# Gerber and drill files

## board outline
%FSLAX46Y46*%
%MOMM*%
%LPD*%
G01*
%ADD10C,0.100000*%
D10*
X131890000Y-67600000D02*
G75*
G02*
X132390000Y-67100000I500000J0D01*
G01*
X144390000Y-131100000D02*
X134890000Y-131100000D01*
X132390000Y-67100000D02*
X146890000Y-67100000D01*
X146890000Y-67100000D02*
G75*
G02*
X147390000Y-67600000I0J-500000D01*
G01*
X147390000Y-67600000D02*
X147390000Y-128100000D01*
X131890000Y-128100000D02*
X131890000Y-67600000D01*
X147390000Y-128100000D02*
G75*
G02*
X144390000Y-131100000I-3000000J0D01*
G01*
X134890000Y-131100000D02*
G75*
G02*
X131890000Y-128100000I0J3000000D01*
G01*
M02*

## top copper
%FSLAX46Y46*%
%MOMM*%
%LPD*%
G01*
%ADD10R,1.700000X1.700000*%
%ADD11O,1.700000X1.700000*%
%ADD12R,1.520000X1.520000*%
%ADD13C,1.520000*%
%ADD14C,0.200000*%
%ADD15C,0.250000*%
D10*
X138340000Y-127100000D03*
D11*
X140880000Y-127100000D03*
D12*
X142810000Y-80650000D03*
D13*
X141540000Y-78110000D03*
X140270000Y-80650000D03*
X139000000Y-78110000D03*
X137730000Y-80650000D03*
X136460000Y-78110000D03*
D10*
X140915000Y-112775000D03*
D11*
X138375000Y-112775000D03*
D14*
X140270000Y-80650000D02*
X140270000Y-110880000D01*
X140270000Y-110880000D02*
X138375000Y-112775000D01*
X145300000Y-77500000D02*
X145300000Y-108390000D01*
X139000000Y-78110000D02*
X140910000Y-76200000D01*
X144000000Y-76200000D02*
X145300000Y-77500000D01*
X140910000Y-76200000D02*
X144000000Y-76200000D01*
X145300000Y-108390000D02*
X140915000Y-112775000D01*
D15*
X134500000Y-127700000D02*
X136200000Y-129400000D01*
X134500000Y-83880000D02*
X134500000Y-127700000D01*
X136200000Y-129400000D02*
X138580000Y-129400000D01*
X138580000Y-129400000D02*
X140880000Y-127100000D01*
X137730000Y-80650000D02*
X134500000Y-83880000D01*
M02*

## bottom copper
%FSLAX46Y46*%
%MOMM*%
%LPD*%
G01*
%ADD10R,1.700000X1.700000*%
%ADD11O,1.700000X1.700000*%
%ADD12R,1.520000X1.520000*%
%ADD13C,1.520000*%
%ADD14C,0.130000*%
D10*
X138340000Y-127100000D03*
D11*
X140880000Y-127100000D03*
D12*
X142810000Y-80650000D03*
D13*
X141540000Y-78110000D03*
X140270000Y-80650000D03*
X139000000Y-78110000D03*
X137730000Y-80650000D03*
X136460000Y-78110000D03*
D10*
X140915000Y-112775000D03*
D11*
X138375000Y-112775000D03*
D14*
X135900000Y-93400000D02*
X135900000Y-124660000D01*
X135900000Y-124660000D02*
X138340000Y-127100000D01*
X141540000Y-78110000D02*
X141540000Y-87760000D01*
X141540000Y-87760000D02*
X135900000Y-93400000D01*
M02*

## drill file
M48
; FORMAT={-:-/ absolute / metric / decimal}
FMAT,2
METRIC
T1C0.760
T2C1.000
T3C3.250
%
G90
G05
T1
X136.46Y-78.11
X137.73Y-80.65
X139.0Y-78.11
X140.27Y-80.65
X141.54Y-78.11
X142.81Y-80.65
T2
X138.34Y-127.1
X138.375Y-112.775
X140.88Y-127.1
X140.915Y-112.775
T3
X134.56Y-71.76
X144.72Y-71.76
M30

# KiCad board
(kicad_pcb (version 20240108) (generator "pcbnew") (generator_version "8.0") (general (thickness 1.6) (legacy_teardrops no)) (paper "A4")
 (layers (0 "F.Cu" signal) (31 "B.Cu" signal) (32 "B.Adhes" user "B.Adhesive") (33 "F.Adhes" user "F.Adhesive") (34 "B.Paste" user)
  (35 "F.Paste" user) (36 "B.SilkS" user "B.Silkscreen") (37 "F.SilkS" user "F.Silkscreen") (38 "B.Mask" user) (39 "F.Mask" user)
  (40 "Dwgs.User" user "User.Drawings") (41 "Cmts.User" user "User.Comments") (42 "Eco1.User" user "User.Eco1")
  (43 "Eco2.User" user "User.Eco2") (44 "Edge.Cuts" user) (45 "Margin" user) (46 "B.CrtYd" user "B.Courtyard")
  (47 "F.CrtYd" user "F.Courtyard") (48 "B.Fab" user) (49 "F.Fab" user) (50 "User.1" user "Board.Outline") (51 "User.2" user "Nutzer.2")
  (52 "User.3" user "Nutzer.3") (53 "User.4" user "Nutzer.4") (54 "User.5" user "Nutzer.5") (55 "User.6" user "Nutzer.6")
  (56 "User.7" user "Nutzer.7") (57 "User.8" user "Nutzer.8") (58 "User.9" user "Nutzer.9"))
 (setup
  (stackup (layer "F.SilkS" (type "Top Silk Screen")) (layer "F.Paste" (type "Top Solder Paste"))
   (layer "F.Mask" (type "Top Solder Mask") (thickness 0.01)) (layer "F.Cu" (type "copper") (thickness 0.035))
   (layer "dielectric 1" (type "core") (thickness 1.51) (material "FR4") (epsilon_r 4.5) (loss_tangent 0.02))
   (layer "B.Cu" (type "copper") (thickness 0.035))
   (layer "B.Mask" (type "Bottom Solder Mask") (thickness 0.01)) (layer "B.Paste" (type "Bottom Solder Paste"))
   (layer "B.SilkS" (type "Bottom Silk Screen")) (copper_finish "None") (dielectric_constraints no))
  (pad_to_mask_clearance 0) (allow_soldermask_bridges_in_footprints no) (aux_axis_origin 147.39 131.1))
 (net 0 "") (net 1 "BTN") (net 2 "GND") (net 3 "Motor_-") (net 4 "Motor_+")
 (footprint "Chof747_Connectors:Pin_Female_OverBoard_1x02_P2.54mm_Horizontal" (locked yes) (layer "F.Cu") (at 138.34 127.1 90)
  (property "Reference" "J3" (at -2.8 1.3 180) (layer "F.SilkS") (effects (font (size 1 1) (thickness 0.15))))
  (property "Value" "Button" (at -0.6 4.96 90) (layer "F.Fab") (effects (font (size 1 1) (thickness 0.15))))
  (pad "1" thru_hole rect (at 0 0 90) (size 1.7 1.7) (drill 1) (layers "*.Cu" "*.Mask") (remove_unused_layers no) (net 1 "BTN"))
  (pad "2" thru_hole oval (at 0 2.54 90) (size 1.7 1.7) (drill 1) (layers "*.Cu" "*.Mask") (remove_unused_layers no) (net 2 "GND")))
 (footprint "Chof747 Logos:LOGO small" (layer "F.Cu") (at 135.099998 91.5)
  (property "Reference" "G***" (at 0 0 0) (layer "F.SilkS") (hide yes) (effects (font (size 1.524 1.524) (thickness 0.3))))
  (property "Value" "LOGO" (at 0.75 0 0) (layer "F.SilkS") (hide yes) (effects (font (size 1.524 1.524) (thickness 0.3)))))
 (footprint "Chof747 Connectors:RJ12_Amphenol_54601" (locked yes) (layer "F.Cu") (at 142.81 80.65 180)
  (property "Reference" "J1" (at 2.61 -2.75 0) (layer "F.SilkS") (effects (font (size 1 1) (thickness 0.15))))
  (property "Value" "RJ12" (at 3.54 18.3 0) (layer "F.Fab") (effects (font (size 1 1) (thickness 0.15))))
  (pad "" np_thru_hole circle (at -1.91 8.89 180) (size 3.25 3.25) (drill 3.25) (layers "*.Cu" "*.Mask"))
  (pad "" np_thru_hole circle (at 8.25 8.89 180) (size 3.25 3.25) (drill 3.25) (layers "*.Cu" "*.Mask"))
  (pad "1" thru_hole rect (at 0 0 180) (size 1.52 1.52) (drill 0.76) (layers "*.Cu" "*.Mask") (remove_unused_layers no))
  (pad "2" thru_hole circle (at 1.27 2.54 180) (size 1.52 1.52) (drill 0.76) (layers "*.Cu" "*.Mask") (remove_unused_layers no)
   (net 1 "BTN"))
  (pad "3" thru_hole circle (at 2.54 0 180) (size 1.52 1.52) (drill 0.76) (layers "*.Cu" "*.Mask") (remove_unused_layers no)
   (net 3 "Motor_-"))
  (pad "4" thru_hole circle (at 3.81 2.54 180) (size 1.52 1.52) (drill 0.76) (layers "*.Cu" "*.Mask") (remove_unused_layers no)
   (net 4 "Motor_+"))
  (pad "5" thru_hole circle (at 5.08 0 180) (size 1.52 1.52) (drill 0.76) (layers "*.Cu" "*.Mask") (remove_unused_layers no) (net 2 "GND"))
  (pad "6" thru_hole circle (at 6.35 2.54 180) (size 1.52 1.52) (drill 0.76) (layers "*.Cu" "*.Mask") (remove_unused_layers no)))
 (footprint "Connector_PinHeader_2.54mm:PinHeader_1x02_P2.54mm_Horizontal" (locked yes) (layer "B.Cu") (at 140.915 112.775 90)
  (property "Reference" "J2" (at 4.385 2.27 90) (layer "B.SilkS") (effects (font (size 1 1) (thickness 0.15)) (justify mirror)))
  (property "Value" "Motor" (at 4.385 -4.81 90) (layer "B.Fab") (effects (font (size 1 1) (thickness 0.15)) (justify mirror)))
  (pad "1" thru_hole rect (at 0 0 90) (size 1.7 1.7) (drill 1) (layers "*.Cu" "*.Mask") (remove_unused_layers no) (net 4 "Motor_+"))
  (pad "2" thru_hole oval (at 0 -2.54 90) (size 1.7 1.7) (drill 1) (layers "*.Cu" "*.Mask") (remove_unused_layers no) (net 3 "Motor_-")))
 (gr_arc (start 131.89 67.6) (mid 132.036447 67.246447) (end 132.39 67.1) (locked yes) (stroke (width 0.1) (type default))
  (layer "Edge.Cuts"))
 (gr_line (start 144.39 131.1) (end 134.89 131.1) (locked yes) (stroke (width 0.1) (type default)) (layer "Edge.Cuts"))
 (gr_line (start 132.39 67.1) (end 146.89 67.1) (locked yes) (stroke (width 0.1) (type default)) (layer "Edge.Cuts"))
 (gr_arc (start 146.89 67.1) (mid 147.243553 67.246447) (end 147.39 67.6) (locked yes) (stroke (width 0.1) (type default))
  (layer "Edge.Cuts"))
 (gr_line (start 147.39 67.6) (end 147.39 128.1) (locked yes) (stroke (width 0.1) (type default)) (layer "Edge.Cuts"))
 (gr_line (start 131.89 128.1) (end 131.89 67.6) (locked yes) (stroke (width 0.1) (type default)) (layer "Edge.Cuts"))
 (gr_arc (start 147.39 128.1) (mid 146.51132 130.22132) (end 144.39 131.1) (locked yes) (stroke (width 0.1) (type default))
  (layer "Edge.Cuts"))
 (gr_arc (start 134.89 131.1) (mid 132.76868 130.22132) (end 131.89 128.1) (locked yes) (stroke (width 0.1) (type default))
  (layer "Edge.Cuts"))
 (segment (start 135.9 93.4) (end 135.9 124.66) (width 0.13) (layer "B.Cu") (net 1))
 (segment (start 135.9 124.66) (end 138.34 127.1) (width 0.13) (layer "B.Cu") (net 1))
 (segment (start 141.54 78.11) (end 141.54 87.76) (width 0.13) (layer "B.Cu") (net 1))
 (segment (start 141.54 87.76) (end 135.9 93.4) (width 0.13) (layer "B.Cu") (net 1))
 (segment (start 140.27 80.65) (end 140.27 110.88) (width 0.2) (layer "F.Cu") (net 3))
 (segment (start 140.27 110.88) (end 138.375 112.775) (width 0.2) (layer "F.Cu") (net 3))
 (segment (start 145.3 77.5) (end 145.3 108.39) (width 0.2) (layer "F.Cu") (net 4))
 (segment (start 139 78.11) (end 140.91 76.2) (width 0.2) (layer "F.Cu") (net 4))
 (segment (start 144 76.2) (end 145.3 77.5) (width 0.2) (layer "F.Cu") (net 4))
 (segment (start 140.91 76.2) (end 144 76.2) (width 0.2) (layer "F.Cu") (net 4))
 (segment (start 145.3 108.39) (end 140.915 112.775) (width 0.2) (layer "F.Cu") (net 4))
 (segment (start 134.5 127.7) (end 136.2 129.4) (width 0.25) (layer "F.Cu") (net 2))
 (segment (start 134.5 83.88) (end 134.5 127.7) (width 0.25) (layer "F.Cu") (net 2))
 (segment (start 136.2 129.4) (end 138.58 129.4) (width 0.25) (layer "F.Cu") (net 2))
 (segment (start 138.58 129.4) (end 140.88 127.1) (width 0.25) (layer "F.Cu") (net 2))
 (segment (start 137.73 80.65) (end 134.5 83.88) (width 0.25) (layer "F.Cu") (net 2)))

